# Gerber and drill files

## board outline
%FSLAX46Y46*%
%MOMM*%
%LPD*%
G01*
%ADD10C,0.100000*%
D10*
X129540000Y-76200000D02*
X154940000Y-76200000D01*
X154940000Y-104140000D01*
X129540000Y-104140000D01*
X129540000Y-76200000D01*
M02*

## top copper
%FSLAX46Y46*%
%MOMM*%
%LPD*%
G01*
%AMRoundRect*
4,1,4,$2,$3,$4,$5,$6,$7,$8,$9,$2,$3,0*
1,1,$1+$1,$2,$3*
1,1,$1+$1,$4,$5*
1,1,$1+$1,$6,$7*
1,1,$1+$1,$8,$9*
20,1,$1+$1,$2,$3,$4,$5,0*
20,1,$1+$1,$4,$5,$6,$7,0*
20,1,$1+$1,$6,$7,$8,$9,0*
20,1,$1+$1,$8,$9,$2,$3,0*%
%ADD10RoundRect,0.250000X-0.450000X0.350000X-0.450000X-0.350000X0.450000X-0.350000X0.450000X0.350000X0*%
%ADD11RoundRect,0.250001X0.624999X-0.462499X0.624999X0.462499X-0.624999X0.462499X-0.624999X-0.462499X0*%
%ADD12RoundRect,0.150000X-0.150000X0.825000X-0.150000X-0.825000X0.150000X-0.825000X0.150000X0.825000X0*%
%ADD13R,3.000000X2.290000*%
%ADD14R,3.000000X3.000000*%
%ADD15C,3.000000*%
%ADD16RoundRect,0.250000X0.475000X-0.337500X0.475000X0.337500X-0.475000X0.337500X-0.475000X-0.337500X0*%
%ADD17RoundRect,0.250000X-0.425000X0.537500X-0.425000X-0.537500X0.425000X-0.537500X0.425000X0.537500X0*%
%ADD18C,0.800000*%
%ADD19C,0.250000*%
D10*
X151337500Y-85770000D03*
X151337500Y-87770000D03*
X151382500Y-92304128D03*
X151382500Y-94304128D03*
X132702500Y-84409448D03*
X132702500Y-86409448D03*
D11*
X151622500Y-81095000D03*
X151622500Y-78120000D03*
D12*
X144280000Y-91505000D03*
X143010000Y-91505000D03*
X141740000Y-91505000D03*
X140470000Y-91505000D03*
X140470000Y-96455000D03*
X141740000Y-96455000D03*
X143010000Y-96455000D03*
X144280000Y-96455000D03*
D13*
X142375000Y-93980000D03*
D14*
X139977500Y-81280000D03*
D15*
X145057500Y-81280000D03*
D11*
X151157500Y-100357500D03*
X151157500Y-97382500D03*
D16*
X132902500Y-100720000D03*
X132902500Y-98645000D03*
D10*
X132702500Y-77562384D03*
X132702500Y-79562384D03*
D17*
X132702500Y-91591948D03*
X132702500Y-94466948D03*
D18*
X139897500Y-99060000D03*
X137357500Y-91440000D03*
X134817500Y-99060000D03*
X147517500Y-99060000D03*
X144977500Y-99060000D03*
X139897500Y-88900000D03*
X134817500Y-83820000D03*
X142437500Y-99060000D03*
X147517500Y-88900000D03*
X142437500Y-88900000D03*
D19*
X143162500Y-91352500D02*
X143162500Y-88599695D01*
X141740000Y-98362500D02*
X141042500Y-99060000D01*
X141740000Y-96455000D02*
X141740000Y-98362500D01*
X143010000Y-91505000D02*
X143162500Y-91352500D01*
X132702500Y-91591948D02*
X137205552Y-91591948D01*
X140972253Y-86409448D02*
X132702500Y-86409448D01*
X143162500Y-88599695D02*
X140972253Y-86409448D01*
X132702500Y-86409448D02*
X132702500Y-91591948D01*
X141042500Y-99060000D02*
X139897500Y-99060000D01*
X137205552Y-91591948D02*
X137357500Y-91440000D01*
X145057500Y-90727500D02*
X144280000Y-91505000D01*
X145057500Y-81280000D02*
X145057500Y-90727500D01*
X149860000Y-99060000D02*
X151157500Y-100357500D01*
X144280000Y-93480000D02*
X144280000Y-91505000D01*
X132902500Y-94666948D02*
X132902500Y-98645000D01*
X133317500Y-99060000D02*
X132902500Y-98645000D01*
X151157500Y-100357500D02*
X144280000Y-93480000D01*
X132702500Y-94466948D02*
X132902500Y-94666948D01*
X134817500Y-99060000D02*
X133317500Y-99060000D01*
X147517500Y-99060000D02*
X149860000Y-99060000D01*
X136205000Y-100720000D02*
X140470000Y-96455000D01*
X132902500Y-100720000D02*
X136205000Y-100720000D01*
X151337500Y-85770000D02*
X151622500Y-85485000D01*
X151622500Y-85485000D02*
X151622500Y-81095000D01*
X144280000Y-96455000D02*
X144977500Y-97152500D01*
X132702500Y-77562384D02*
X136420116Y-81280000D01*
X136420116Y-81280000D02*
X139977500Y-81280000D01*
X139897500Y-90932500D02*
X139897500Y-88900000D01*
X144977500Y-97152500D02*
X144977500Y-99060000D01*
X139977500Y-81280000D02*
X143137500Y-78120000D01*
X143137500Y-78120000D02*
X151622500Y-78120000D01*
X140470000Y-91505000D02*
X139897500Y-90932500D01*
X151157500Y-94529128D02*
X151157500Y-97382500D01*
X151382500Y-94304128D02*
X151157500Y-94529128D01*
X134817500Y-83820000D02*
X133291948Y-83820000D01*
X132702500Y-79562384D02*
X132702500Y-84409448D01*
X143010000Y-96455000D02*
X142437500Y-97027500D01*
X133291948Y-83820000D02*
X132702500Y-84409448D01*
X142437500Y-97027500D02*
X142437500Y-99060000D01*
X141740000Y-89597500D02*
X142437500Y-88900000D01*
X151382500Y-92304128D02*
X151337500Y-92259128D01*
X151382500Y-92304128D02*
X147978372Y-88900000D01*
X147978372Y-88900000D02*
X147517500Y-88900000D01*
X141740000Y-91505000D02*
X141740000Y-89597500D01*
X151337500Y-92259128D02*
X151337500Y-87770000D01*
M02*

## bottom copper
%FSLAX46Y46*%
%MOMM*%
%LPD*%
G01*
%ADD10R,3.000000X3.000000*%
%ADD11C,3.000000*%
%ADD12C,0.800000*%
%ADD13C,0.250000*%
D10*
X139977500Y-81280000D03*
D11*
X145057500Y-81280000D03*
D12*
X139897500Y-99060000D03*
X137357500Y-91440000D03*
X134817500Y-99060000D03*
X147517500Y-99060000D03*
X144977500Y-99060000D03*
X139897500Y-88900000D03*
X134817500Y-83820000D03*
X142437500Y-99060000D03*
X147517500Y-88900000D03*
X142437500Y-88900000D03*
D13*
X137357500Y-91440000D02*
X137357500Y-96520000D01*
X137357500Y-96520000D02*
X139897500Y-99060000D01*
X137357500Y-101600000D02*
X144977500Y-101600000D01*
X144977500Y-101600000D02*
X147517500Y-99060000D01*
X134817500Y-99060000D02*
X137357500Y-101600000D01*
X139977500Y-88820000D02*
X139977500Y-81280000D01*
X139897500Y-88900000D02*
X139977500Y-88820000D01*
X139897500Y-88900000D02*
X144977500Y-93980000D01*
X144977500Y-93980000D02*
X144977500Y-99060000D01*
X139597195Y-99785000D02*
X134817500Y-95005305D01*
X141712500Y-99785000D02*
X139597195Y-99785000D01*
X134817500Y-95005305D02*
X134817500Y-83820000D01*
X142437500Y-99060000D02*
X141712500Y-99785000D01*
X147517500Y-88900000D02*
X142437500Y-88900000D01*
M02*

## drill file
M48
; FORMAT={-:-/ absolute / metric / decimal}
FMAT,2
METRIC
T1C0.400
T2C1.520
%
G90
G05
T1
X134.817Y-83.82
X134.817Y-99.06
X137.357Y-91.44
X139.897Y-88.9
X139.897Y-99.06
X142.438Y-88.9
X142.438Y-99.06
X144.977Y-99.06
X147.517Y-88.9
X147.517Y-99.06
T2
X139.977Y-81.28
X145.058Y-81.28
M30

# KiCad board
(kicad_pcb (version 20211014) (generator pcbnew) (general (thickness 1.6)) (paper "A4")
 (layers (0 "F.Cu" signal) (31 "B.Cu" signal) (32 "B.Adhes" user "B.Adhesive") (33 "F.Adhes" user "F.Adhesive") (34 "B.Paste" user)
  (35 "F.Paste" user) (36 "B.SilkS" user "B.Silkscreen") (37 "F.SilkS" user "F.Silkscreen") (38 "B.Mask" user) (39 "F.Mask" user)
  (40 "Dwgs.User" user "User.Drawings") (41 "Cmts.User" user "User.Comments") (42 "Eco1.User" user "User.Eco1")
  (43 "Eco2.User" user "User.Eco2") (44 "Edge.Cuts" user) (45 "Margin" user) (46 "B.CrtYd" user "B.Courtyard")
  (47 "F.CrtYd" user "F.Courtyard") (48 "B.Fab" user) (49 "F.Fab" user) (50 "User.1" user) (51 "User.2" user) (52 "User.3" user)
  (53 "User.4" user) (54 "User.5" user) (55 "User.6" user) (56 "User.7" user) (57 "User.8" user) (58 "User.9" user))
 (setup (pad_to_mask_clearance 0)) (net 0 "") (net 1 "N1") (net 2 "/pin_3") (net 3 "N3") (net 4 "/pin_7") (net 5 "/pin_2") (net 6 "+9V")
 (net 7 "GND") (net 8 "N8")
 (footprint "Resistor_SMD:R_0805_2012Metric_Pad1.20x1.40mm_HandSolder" (layer "F.Cu") (at 151.3375 86.77 -90)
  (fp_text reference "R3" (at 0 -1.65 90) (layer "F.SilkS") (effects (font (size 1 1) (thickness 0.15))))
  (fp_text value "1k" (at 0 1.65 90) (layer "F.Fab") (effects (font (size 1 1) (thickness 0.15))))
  (pad "1" smd roundrect (at -1 0 270) (size 1.2 1.4) (layers "F.Cu" "F.Paste" "F.Mask") (roundrect_rratio 0.208333) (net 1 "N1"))
  (pad "2" smd roundrect (at 1 0 270) (size 1.2 1.4) (layers "F.Cu" "F.Paste" "F.Mask") (roundrect_rratio 0.208333) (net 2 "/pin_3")))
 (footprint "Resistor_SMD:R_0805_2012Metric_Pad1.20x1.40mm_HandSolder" (layer "F.Cu") (at 151.3825 93.304128 -90)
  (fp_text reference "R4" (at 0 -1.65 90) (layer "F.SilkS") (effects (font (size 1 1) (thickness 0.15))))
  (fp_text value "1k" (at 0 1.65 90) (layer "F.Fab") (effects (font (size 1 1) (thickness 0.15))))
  (pad "1" smd roundrect (at -1 0 270) (size 1.2 1.4) (layers "F.Cu" "F.Paste" "F.Mask") (roundrect_rratio 0.208333) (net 2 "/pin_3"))
  (pad "2" smd roundrect (at 1 0 270) (size 1.2 1.4) (layers "F.Cu" "F.Paste" "F.Mask") (roundrect_rratio 0.208333) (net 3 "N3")))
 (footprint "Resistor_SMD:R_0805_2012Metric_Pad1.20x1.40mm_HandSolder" (layer "F.Cu") (at 132.7025 85.409448 -90)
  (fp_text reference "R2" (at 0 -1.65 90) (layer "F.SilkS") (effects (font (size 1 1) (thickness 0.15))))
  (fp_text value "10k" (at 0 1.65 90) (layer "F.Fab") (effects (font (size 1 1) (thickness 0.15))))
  (pad "1" smd roundrect (at -1 0 270) (size 1.2 1.4) (layers "F.Cu" "F.Paste" "F.Mask") (roundrect_rratio 0.208333) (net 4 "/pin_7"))
  (pad "2" smd roundrect (at 1 0 270) (size 1.2 1.4) (layers "F.Cu" "F.Paste" "F.Mask") (roundrect_rratio 0.208333) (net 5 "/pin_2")))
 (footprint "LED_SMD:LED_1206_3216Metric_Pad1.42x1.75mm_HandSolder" (layer "F.Cu") (at 151.6225 79.6075 90)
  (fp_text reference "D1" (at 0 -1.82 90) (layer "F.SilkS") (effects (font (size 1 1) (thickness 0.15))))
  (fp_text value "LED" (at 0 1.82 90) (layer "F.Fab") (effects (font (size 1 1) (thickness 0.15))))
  (pad "1" smd roundrect (at -1.4875 0 90) (size 1.425 1.75) (layers "F.Cu" "F.Paste" "F.Mask") (roundrect_rratio 0.175439) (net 1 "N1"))
  (pad "2" smd roundrect (at 1.4875 0 90) (size 1.425 1.75) (layers "F.Cu" "F.Paste" "F.Mask") (roundrect_rratio 0.175439) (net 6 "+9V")))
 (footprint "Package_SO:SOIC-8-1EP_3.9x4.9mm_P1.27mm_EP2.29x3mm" (layer "F.Cu") (at 142.375 93.98 -90)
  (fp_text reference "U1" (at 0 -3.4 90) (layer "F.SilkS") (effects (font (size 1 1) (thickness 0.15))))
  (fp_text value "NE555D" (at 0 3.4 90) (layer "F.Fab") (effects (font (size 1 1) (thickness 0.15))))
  (pad "" smd roundrect (at -0.57 -0.75 270) (size 0.92 1.21) (layers "F.Paste") (roundrect_rratio 0.25))
  (pad "" smd roundrect (at 0.57 0.75 270) (size 0.92 1.21) (layers "F.Paste") (roundrect_rratio 0.25))
  (pad "" smd roundrect (at 0.57 -0.75 270) (size 0.92 1.21) (layers "F.Paste") (roundrect_rratio 0.25))
  (pad "" smd roundrect (at -0.57 0.75 270) (size 0.92 1.21) (layers "F.Paste") (roundrect_rratio 0.25))
  (pad "1" smd roundrect (at -2.475 -1.905 270) (size 1.95 0.6) (layers "F.Cu" "F.Paste" "F.Mask") (roundrect_rratio 0.25) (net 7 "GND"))
  (pad "2" smd roundrect (at -2.475 -0.635 270) (size 1.95 0.6) (layers "F.Cu" "F.Paste" "F.Mask") (roundrect_rratio 0.25) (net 5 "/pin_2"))
  (pad "3" smd roundrect (at -2.475 0.635 270) (size 1.95 0.6) (layers "F.Cu" "F.Paste" "F.Mask") (roundrect_rratio 0.25) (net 2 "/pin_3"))
  (pad "4" smd roundrect (at -2.475 1.905 270) (size 1.95 0.6) (layers "F.Cu" "F.Paste" "F.Mask") (roundrect_rratio 0.25) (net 6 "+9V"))
  (pad "5" smd roundrect (at 2.475 1.905 270) (size 1.95 0.6) (layers "F.Cu" "F.Paste" "F.Mask") (roundrect_rratio 0.25) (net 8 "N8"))
  (pad "6" smd roundrect (at 2.475 0.635 270) (size 1.95 0.6) (layers "F.Cu" "F.Paste" "F.Mask") (roundrect_rratio 0.25) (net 5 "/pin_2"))
  (pad "7" smd roundrect (at 2.475 -0.635 270) (size 1.95 0.6) (layers "F.Cu" "F.Paste" "F.Mask") (roundrect_rratio 0.25) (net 4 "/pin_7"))
  (pad "8" smd roundrect (at 2.475 -1.905 270) (size 1.95 0.6) (layers "F.Cu" "F.Paste" "F.Mask") (roundrect_rratio 0.25) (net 6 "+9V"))
  (pad "9" smd rect (at 0 0 270) (size 2.29 3) (layers "F.Cu" "F.Mask")))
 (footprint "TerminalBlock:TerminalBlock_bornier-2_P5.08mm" (layer "F.Cu") (at 139.9775 81.28)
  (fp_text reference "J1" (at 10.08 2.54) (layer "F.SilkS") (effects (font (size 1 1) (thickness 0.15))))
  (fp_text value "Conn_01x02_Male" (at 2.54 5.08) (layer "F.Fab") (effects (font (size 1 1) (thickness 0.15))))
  (pad "1" thru_hole rect (at 0 0) (size 3 3) (drill 1.52) (layers *.Cu *.Mask) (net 6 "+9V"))
  (pad "2" thru_hole circle (at 5.08 0) (size 3 3) (drill 1.52) (layers *.Cu *.Mask) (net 7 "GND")))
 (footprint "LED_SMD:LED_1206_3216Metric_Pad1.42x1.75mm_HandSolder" (layer "F.Cu") (at 151.1575 98.87 90)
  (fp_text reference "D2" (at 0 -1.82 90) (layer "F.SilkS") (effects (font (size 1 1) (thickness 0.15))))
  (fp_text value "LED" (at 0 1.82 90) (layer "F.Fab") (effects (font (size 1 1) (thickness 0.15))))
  (pad "1" smd roundrect (at -1.4875 0 90) (size 1.425 1.75) (layers "F.Cu" "F.Paste" "F.Mask") (roundrect_rratio 0.175439) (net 7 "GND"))
  (pad "2" smd roundrect (at 1.4875 0 90) (size 1.425 1.75) (layers "F.Cu" "F.Paste" "F.Mask") (roundrect_rratio 0.175439) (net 3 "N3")))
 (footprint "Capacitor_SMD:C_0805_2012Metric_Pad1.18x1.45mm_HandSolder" (layer "F.Cu") (at 132.9025 99.6825 90)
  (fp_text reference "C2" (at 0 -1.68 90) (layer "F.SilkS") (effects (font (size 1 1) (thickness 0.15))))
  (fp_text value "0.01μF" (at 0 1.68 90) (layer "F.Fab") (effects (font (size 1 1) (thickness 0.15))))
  (pad "1" smd roundrect (at -1.0375 0 90) (size 1.175 1.45) (layers "F.Cu" "F.Paste" "F.Mask") (roundrect_rratio 0.212766) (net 8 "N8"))
  (pad "2" smd roundrect (at 1.0375 0 90) (size 1.175 1.45) (layers "F.Cu" "F.Paste" "F.Mask") (roundrect_rratio 0.212766) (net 7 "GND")))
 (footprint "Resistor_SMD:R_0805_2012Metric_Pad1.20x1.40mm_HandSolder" (layer "F.Cu") (at 132.7025 78.562384 -90)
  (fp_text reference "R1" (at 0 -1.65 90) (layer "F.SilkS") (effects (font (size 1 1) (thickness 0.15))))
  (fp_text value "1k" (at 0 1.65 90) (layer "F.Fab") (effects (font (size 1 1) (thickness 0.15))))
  (pad "1" smd roundrect (at -1 0 270) (size 1.2 1.4) (layers "F.Cu" "F.Paste" "F.Mask") (roundrect_rratio 0.208333) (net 6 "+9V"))
  (pad "2" smd roundrect (at 1 0 270) (size 1.2 1.4) (layers "F.Cu" "F.Paste" "F.Mask") (roundrect_rratio 0.208333) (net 4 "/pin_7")))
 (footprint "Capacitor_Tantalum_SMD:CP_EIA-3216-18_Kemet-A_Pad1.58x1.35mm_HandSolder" (layer "F.Cu") (at 132.7025 93.029448 -90)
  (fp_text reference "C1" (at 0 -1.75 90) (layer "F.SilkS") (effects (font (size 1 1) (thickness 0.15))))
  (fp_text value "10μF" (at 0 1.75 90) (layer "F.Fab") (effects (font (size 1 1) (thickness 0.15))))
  (pad "1" smd roundrect (at -1.4375 0 270) (size 1.575 1.35) (layers "F.Cu" "F.Paste" "F.Mask") (roundrect_rratio 0.185185)
   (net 5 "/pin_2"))
  (pad "2" smd roundrect (at 1.4375 0 270) (size 1.575 1.35) (layers "F.Cu" "F.Paste" "F.Mask") (roundrect_rratio 0.185185) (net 7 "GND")))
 (gr_rect (start 129.54 76.2) (end 154.94 104.14) (layer "Edge.Cuts") (width 0.1) (fill none))
 (segment (start 143.1625 91.3525) (end 143.1625 88.599695) (width 0.25) (layer "F.Cu") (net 5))
 (segment (start 141.74 98.3625) (end 141.0425 99.06) (width 0.25) (layer "F.Cu") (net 5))
 (segment (start 141.74 96.455) (end 141.74 98.3625) (width 0.25) (layer "F.Cu") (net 5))
 (segment (start 143.01 91.505) (end 143.1625 91.3525) (width 0.25) (layer "F.Cu") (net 5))
 (segment (start 132.7025 91.591948) (end 137.205552 91.591948) (width 0.25) (layer "F.Cu") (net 5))
 (segment (start 140.972253 86.409448) (end 132.7025 86.409448) (width 0.25) (layer "F.Cu") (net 5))
 (segment (start 143.1625 88.599695) (end 140.972253 86.409448) (width 0.25) (layer "F.Cu") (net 5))
 (segment (start 132.7025 86.409448) (end 132.7025 91.591948) (width 0.25) (layer "F.Cu") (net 5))
 (segment (start 141.0425 99.06) (end 139.8975 99.06) (width 0.25) (layer "F.Cu") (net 5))
 (segment (start 137.205552 91.591948) (end 137.3575 91.44) (width 0.25) (layer "F.Cu") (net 5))
 (via (at 139.8975 99.06) (size 0.8) (drill 0.4) (layers "F.Cu" "B.Cu") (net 5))
 (via (at 137.3575 91.44) (size 0.8) (drill 0.4) (layers "F.Cu" "B.Cu") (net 5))
 (segment (start 137.3575 91.44) (end 137.3575 96.52) (width 0.25) (layer "B.Cu") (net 5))
 (segment (start 137.3575 96.52) (end 139.8975 99.06) (width 0.25) (layer "B.Cu") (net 5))
 (segment (start 145.0575 90.7275) (end 144.28 91.505) (width 0.25) (layer "F.Cu") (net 7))
 (segment (start 145.0575 81.28) (end 145.0575 90.7275) (width 0.25) (layer "F.Cu") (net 7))
 (segment (start 149.86 99.06) (end 151.1575 100.3575) (width 0.25) (layer "F.Cu") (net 7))
 (segment (start 144.28 93.48) (end 144.28 91.505) (width 0.25) (layer "F.Cu") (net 7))
 (segment (start 132.9025 94.666948) (end 132.9025 98.645) (width 0.25) (layer "F.Cu") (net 7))
 (segment (start 133.3175 99.06) (end 132.9025 98.645) (width 0.25) (layer "F.Cu") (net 7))
 (segment (start 151.1575 100.3575) (end 144.28 93.48) (width 0.25) (layer "F.Cu") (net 7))
 (segment (start 132.7025 94.466948) (end 132.9025 94.666948) (width 0.25) (layer "F.Cu") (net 7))
 (segment (start 134.8175 99.06) (end 133.3175 99.06) (width 0.25) (layer "F.Cu") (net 7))
 (segment (start 147.5175 99.06) (end 149.86 99.06) (width 0.25) (layer "F.Cu") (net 7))
 (via (at 134.8175 99.06) (size 0.8) (drill 0.4) (layers "F.Cu" "B.Cu") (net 7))
 (via (at 147.5175 99.06) (size 0.8) (drill 0.4) (layers "F.Cu" "B.Cu") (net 7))
 (segment (start 137.3575 101.6) (end 144.9775 101.6) (width 0.25) (layer "B.Cu") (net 7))
 (segment (start 144.9775 101.6) (end 147.5175 99.06) (width 0.25) (layer "B.Cu") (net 7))
 (segment (start 134.8175 99.06) (end 137.3575 101.6) (width 0.25) (layer "B.Cu") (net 7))
 (segment (start 136.205 100.72) (end 140.47 96.455) (width 0.25) (layer "F.Cu") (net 8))
 (segment (start 132.9025 100.72) (end 136.205 100.72) (width 0.25) (layer "F.Cu") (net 8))
 (segment (start 151.3375 85.77) (end 151.6225 85.485) (width 0.25) (layer "F.Cu") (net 1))
 (segment (start 151.6225 85.485) (end 151.6225 81.095) (width 0.25) (layer "F.Cu") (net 1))
 (segment (start 144.28 96.455) (end 144.9775 97.1525) (width 0.25) (layer "F.Cu") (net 6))
 (segment (start 132.7025 77.562384) (end 136.420116 81.28) (width 0.25) (layer "F.Cu") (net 6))
 (segment (start 136.420116 81.28) (end 139.9775 81.28) (width 0.25) (layer "F.Cu") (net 6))
 (segment (start 139.8975 90.9325) (end 139.8975 88.9) (width 0.25) (layer "F.Cu") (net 6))
 (segment (start 144.9775 97.1525) (end 144.9775 99.06) (width 0.25) (layer "F.Cu") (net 6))
 (segment (start 139.9775 81.28) (end 143.1375 78.12) (width 0.25) (layer "F.Cu") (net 6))
 (segment (start 143.1375 78.12) (end 151.6225 78.12) (width 0.25) (layer "F.Cu") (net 6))
 (segment (start 140.47 91.505) (end 139.8975 90.9325) (width 0.25) (layer "F.Cu") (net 6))
 (via (at 144.9775 99.06) (size 0.8) (drill 0.4) (layers "F.Cu" "B.Cu") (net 6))
 (via (at 139.8975 88.9) (size 0.8) (drill 0.4) (layers "F.Cu" "B.Cu") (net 6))
 (segment (start 139.9775 88.82) (end 139.9775 81.28) (width 0.25) (layer "B.Cu") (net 6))
 (segment (start 139.8975 88.9) (end 139.9775 88.82) (width 0.25) (layer "B.Cu") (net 6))
 (segment (start 139.8975 88.9) (end 144.9775 93.98) (width 0.25) (layer "B.Cu") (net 6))
 (segment (start 144.9775 93.98) (end 144.9775 99.06) (width 0.25) (layer "B.Cu") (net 6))
 (segment (start 151.1575 94.529128) (end 151.1575 97.3825) (width 0.25) (layer "F.Cu") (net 3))
 (segment (start 151.3825 94.304128) (end 151.1575 94.529128) (width 0.25) (layer "F.Cu") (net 3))
 (segment (start 134.8175 83.82) (end 133.291948 83.82) (width 0.25) (layer "F.Cu") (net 4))
 (segment (start 132.7025 79.562384) (end 132.7025 84.409448) (width 0.25) (layer "F.Cu") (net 4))
 (segment (start 143.01 96.455) (end 142.4375 97.0275) (width 0.25) (layer "F.Cu") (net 4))
 (segment (start 133.291948 83.82) (end 132.7025 84.409448) (width 0.25) (layer "F.Cu") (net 4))
 (segment (start 142.4375 97.0275) (end 142.4375 99.06) (width 0.25) (layer "F.Cu") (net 4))
 (via (at 134.8175 83.82) (size 0.8) (drill 0.4) (layers "F.Cu" "B.Cu") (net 4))
 (via (at 142.4375 99.06) (size 0.8) (drill 0.4) (layers "F.Cu" "B.Cu") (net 4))
 (segment (start 139.597195 99.785) (end 134.8175 95.005305) (width 0.25) (layer "B.Cu") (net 4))
 (segment (start 141.7125 99.785) (end 139.597195 99.785) (width 0.25) (layer "B.Cu") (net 4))
 (segment (start 134.8175 95.005305) (end 134.8175 83.82) (width 0.25) (layer "B.Cu") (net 4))
 (segment (start 142.4375 99.06) (end 141.7125 99.785) (width 0.25) (layer "B.Cu") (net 4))
 (segment (start 141.74 89.5975) (end 142.4375 88.9) (width 0.25) (layer "F.Cu") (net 2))
 (segment (start 151.3825 92.304128) (end 151.3375 92.259128) (width 0.25) (layer "F.Cu") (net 2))
 (segment (start 151.3825 92.304128) (end 147.978372 88.9) (width 0.25) (layer "F.Cu") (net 2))
 (segment (start 147.978372 88.9) (end 147.5175 88.9) (width 0.25) (layer "F.Cu") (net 2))
 (segment (start 141.74 91.505) (end 141.74 89.5975) (width 0.25) (layer "F.Cu") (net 2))
 (segment (start 151.3375 92.259128) (end 151.3375 87.77) (width 0.25) (layer "F.Cu") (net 2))
 (via (at 147.5175 88.9) (size 0.8) (drill 0.4) (layers "F.Cu" "B.Cu") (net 2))
 (via (at 142.4375 88.9) (size 0.8) (drill 0.4) (layers "F.Cu" "B.Cu") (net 2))
 (segment (start 147.5175 88.9) (end 142.4375 88.9) (width 0.25) (layer "B.Cu") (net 2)))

